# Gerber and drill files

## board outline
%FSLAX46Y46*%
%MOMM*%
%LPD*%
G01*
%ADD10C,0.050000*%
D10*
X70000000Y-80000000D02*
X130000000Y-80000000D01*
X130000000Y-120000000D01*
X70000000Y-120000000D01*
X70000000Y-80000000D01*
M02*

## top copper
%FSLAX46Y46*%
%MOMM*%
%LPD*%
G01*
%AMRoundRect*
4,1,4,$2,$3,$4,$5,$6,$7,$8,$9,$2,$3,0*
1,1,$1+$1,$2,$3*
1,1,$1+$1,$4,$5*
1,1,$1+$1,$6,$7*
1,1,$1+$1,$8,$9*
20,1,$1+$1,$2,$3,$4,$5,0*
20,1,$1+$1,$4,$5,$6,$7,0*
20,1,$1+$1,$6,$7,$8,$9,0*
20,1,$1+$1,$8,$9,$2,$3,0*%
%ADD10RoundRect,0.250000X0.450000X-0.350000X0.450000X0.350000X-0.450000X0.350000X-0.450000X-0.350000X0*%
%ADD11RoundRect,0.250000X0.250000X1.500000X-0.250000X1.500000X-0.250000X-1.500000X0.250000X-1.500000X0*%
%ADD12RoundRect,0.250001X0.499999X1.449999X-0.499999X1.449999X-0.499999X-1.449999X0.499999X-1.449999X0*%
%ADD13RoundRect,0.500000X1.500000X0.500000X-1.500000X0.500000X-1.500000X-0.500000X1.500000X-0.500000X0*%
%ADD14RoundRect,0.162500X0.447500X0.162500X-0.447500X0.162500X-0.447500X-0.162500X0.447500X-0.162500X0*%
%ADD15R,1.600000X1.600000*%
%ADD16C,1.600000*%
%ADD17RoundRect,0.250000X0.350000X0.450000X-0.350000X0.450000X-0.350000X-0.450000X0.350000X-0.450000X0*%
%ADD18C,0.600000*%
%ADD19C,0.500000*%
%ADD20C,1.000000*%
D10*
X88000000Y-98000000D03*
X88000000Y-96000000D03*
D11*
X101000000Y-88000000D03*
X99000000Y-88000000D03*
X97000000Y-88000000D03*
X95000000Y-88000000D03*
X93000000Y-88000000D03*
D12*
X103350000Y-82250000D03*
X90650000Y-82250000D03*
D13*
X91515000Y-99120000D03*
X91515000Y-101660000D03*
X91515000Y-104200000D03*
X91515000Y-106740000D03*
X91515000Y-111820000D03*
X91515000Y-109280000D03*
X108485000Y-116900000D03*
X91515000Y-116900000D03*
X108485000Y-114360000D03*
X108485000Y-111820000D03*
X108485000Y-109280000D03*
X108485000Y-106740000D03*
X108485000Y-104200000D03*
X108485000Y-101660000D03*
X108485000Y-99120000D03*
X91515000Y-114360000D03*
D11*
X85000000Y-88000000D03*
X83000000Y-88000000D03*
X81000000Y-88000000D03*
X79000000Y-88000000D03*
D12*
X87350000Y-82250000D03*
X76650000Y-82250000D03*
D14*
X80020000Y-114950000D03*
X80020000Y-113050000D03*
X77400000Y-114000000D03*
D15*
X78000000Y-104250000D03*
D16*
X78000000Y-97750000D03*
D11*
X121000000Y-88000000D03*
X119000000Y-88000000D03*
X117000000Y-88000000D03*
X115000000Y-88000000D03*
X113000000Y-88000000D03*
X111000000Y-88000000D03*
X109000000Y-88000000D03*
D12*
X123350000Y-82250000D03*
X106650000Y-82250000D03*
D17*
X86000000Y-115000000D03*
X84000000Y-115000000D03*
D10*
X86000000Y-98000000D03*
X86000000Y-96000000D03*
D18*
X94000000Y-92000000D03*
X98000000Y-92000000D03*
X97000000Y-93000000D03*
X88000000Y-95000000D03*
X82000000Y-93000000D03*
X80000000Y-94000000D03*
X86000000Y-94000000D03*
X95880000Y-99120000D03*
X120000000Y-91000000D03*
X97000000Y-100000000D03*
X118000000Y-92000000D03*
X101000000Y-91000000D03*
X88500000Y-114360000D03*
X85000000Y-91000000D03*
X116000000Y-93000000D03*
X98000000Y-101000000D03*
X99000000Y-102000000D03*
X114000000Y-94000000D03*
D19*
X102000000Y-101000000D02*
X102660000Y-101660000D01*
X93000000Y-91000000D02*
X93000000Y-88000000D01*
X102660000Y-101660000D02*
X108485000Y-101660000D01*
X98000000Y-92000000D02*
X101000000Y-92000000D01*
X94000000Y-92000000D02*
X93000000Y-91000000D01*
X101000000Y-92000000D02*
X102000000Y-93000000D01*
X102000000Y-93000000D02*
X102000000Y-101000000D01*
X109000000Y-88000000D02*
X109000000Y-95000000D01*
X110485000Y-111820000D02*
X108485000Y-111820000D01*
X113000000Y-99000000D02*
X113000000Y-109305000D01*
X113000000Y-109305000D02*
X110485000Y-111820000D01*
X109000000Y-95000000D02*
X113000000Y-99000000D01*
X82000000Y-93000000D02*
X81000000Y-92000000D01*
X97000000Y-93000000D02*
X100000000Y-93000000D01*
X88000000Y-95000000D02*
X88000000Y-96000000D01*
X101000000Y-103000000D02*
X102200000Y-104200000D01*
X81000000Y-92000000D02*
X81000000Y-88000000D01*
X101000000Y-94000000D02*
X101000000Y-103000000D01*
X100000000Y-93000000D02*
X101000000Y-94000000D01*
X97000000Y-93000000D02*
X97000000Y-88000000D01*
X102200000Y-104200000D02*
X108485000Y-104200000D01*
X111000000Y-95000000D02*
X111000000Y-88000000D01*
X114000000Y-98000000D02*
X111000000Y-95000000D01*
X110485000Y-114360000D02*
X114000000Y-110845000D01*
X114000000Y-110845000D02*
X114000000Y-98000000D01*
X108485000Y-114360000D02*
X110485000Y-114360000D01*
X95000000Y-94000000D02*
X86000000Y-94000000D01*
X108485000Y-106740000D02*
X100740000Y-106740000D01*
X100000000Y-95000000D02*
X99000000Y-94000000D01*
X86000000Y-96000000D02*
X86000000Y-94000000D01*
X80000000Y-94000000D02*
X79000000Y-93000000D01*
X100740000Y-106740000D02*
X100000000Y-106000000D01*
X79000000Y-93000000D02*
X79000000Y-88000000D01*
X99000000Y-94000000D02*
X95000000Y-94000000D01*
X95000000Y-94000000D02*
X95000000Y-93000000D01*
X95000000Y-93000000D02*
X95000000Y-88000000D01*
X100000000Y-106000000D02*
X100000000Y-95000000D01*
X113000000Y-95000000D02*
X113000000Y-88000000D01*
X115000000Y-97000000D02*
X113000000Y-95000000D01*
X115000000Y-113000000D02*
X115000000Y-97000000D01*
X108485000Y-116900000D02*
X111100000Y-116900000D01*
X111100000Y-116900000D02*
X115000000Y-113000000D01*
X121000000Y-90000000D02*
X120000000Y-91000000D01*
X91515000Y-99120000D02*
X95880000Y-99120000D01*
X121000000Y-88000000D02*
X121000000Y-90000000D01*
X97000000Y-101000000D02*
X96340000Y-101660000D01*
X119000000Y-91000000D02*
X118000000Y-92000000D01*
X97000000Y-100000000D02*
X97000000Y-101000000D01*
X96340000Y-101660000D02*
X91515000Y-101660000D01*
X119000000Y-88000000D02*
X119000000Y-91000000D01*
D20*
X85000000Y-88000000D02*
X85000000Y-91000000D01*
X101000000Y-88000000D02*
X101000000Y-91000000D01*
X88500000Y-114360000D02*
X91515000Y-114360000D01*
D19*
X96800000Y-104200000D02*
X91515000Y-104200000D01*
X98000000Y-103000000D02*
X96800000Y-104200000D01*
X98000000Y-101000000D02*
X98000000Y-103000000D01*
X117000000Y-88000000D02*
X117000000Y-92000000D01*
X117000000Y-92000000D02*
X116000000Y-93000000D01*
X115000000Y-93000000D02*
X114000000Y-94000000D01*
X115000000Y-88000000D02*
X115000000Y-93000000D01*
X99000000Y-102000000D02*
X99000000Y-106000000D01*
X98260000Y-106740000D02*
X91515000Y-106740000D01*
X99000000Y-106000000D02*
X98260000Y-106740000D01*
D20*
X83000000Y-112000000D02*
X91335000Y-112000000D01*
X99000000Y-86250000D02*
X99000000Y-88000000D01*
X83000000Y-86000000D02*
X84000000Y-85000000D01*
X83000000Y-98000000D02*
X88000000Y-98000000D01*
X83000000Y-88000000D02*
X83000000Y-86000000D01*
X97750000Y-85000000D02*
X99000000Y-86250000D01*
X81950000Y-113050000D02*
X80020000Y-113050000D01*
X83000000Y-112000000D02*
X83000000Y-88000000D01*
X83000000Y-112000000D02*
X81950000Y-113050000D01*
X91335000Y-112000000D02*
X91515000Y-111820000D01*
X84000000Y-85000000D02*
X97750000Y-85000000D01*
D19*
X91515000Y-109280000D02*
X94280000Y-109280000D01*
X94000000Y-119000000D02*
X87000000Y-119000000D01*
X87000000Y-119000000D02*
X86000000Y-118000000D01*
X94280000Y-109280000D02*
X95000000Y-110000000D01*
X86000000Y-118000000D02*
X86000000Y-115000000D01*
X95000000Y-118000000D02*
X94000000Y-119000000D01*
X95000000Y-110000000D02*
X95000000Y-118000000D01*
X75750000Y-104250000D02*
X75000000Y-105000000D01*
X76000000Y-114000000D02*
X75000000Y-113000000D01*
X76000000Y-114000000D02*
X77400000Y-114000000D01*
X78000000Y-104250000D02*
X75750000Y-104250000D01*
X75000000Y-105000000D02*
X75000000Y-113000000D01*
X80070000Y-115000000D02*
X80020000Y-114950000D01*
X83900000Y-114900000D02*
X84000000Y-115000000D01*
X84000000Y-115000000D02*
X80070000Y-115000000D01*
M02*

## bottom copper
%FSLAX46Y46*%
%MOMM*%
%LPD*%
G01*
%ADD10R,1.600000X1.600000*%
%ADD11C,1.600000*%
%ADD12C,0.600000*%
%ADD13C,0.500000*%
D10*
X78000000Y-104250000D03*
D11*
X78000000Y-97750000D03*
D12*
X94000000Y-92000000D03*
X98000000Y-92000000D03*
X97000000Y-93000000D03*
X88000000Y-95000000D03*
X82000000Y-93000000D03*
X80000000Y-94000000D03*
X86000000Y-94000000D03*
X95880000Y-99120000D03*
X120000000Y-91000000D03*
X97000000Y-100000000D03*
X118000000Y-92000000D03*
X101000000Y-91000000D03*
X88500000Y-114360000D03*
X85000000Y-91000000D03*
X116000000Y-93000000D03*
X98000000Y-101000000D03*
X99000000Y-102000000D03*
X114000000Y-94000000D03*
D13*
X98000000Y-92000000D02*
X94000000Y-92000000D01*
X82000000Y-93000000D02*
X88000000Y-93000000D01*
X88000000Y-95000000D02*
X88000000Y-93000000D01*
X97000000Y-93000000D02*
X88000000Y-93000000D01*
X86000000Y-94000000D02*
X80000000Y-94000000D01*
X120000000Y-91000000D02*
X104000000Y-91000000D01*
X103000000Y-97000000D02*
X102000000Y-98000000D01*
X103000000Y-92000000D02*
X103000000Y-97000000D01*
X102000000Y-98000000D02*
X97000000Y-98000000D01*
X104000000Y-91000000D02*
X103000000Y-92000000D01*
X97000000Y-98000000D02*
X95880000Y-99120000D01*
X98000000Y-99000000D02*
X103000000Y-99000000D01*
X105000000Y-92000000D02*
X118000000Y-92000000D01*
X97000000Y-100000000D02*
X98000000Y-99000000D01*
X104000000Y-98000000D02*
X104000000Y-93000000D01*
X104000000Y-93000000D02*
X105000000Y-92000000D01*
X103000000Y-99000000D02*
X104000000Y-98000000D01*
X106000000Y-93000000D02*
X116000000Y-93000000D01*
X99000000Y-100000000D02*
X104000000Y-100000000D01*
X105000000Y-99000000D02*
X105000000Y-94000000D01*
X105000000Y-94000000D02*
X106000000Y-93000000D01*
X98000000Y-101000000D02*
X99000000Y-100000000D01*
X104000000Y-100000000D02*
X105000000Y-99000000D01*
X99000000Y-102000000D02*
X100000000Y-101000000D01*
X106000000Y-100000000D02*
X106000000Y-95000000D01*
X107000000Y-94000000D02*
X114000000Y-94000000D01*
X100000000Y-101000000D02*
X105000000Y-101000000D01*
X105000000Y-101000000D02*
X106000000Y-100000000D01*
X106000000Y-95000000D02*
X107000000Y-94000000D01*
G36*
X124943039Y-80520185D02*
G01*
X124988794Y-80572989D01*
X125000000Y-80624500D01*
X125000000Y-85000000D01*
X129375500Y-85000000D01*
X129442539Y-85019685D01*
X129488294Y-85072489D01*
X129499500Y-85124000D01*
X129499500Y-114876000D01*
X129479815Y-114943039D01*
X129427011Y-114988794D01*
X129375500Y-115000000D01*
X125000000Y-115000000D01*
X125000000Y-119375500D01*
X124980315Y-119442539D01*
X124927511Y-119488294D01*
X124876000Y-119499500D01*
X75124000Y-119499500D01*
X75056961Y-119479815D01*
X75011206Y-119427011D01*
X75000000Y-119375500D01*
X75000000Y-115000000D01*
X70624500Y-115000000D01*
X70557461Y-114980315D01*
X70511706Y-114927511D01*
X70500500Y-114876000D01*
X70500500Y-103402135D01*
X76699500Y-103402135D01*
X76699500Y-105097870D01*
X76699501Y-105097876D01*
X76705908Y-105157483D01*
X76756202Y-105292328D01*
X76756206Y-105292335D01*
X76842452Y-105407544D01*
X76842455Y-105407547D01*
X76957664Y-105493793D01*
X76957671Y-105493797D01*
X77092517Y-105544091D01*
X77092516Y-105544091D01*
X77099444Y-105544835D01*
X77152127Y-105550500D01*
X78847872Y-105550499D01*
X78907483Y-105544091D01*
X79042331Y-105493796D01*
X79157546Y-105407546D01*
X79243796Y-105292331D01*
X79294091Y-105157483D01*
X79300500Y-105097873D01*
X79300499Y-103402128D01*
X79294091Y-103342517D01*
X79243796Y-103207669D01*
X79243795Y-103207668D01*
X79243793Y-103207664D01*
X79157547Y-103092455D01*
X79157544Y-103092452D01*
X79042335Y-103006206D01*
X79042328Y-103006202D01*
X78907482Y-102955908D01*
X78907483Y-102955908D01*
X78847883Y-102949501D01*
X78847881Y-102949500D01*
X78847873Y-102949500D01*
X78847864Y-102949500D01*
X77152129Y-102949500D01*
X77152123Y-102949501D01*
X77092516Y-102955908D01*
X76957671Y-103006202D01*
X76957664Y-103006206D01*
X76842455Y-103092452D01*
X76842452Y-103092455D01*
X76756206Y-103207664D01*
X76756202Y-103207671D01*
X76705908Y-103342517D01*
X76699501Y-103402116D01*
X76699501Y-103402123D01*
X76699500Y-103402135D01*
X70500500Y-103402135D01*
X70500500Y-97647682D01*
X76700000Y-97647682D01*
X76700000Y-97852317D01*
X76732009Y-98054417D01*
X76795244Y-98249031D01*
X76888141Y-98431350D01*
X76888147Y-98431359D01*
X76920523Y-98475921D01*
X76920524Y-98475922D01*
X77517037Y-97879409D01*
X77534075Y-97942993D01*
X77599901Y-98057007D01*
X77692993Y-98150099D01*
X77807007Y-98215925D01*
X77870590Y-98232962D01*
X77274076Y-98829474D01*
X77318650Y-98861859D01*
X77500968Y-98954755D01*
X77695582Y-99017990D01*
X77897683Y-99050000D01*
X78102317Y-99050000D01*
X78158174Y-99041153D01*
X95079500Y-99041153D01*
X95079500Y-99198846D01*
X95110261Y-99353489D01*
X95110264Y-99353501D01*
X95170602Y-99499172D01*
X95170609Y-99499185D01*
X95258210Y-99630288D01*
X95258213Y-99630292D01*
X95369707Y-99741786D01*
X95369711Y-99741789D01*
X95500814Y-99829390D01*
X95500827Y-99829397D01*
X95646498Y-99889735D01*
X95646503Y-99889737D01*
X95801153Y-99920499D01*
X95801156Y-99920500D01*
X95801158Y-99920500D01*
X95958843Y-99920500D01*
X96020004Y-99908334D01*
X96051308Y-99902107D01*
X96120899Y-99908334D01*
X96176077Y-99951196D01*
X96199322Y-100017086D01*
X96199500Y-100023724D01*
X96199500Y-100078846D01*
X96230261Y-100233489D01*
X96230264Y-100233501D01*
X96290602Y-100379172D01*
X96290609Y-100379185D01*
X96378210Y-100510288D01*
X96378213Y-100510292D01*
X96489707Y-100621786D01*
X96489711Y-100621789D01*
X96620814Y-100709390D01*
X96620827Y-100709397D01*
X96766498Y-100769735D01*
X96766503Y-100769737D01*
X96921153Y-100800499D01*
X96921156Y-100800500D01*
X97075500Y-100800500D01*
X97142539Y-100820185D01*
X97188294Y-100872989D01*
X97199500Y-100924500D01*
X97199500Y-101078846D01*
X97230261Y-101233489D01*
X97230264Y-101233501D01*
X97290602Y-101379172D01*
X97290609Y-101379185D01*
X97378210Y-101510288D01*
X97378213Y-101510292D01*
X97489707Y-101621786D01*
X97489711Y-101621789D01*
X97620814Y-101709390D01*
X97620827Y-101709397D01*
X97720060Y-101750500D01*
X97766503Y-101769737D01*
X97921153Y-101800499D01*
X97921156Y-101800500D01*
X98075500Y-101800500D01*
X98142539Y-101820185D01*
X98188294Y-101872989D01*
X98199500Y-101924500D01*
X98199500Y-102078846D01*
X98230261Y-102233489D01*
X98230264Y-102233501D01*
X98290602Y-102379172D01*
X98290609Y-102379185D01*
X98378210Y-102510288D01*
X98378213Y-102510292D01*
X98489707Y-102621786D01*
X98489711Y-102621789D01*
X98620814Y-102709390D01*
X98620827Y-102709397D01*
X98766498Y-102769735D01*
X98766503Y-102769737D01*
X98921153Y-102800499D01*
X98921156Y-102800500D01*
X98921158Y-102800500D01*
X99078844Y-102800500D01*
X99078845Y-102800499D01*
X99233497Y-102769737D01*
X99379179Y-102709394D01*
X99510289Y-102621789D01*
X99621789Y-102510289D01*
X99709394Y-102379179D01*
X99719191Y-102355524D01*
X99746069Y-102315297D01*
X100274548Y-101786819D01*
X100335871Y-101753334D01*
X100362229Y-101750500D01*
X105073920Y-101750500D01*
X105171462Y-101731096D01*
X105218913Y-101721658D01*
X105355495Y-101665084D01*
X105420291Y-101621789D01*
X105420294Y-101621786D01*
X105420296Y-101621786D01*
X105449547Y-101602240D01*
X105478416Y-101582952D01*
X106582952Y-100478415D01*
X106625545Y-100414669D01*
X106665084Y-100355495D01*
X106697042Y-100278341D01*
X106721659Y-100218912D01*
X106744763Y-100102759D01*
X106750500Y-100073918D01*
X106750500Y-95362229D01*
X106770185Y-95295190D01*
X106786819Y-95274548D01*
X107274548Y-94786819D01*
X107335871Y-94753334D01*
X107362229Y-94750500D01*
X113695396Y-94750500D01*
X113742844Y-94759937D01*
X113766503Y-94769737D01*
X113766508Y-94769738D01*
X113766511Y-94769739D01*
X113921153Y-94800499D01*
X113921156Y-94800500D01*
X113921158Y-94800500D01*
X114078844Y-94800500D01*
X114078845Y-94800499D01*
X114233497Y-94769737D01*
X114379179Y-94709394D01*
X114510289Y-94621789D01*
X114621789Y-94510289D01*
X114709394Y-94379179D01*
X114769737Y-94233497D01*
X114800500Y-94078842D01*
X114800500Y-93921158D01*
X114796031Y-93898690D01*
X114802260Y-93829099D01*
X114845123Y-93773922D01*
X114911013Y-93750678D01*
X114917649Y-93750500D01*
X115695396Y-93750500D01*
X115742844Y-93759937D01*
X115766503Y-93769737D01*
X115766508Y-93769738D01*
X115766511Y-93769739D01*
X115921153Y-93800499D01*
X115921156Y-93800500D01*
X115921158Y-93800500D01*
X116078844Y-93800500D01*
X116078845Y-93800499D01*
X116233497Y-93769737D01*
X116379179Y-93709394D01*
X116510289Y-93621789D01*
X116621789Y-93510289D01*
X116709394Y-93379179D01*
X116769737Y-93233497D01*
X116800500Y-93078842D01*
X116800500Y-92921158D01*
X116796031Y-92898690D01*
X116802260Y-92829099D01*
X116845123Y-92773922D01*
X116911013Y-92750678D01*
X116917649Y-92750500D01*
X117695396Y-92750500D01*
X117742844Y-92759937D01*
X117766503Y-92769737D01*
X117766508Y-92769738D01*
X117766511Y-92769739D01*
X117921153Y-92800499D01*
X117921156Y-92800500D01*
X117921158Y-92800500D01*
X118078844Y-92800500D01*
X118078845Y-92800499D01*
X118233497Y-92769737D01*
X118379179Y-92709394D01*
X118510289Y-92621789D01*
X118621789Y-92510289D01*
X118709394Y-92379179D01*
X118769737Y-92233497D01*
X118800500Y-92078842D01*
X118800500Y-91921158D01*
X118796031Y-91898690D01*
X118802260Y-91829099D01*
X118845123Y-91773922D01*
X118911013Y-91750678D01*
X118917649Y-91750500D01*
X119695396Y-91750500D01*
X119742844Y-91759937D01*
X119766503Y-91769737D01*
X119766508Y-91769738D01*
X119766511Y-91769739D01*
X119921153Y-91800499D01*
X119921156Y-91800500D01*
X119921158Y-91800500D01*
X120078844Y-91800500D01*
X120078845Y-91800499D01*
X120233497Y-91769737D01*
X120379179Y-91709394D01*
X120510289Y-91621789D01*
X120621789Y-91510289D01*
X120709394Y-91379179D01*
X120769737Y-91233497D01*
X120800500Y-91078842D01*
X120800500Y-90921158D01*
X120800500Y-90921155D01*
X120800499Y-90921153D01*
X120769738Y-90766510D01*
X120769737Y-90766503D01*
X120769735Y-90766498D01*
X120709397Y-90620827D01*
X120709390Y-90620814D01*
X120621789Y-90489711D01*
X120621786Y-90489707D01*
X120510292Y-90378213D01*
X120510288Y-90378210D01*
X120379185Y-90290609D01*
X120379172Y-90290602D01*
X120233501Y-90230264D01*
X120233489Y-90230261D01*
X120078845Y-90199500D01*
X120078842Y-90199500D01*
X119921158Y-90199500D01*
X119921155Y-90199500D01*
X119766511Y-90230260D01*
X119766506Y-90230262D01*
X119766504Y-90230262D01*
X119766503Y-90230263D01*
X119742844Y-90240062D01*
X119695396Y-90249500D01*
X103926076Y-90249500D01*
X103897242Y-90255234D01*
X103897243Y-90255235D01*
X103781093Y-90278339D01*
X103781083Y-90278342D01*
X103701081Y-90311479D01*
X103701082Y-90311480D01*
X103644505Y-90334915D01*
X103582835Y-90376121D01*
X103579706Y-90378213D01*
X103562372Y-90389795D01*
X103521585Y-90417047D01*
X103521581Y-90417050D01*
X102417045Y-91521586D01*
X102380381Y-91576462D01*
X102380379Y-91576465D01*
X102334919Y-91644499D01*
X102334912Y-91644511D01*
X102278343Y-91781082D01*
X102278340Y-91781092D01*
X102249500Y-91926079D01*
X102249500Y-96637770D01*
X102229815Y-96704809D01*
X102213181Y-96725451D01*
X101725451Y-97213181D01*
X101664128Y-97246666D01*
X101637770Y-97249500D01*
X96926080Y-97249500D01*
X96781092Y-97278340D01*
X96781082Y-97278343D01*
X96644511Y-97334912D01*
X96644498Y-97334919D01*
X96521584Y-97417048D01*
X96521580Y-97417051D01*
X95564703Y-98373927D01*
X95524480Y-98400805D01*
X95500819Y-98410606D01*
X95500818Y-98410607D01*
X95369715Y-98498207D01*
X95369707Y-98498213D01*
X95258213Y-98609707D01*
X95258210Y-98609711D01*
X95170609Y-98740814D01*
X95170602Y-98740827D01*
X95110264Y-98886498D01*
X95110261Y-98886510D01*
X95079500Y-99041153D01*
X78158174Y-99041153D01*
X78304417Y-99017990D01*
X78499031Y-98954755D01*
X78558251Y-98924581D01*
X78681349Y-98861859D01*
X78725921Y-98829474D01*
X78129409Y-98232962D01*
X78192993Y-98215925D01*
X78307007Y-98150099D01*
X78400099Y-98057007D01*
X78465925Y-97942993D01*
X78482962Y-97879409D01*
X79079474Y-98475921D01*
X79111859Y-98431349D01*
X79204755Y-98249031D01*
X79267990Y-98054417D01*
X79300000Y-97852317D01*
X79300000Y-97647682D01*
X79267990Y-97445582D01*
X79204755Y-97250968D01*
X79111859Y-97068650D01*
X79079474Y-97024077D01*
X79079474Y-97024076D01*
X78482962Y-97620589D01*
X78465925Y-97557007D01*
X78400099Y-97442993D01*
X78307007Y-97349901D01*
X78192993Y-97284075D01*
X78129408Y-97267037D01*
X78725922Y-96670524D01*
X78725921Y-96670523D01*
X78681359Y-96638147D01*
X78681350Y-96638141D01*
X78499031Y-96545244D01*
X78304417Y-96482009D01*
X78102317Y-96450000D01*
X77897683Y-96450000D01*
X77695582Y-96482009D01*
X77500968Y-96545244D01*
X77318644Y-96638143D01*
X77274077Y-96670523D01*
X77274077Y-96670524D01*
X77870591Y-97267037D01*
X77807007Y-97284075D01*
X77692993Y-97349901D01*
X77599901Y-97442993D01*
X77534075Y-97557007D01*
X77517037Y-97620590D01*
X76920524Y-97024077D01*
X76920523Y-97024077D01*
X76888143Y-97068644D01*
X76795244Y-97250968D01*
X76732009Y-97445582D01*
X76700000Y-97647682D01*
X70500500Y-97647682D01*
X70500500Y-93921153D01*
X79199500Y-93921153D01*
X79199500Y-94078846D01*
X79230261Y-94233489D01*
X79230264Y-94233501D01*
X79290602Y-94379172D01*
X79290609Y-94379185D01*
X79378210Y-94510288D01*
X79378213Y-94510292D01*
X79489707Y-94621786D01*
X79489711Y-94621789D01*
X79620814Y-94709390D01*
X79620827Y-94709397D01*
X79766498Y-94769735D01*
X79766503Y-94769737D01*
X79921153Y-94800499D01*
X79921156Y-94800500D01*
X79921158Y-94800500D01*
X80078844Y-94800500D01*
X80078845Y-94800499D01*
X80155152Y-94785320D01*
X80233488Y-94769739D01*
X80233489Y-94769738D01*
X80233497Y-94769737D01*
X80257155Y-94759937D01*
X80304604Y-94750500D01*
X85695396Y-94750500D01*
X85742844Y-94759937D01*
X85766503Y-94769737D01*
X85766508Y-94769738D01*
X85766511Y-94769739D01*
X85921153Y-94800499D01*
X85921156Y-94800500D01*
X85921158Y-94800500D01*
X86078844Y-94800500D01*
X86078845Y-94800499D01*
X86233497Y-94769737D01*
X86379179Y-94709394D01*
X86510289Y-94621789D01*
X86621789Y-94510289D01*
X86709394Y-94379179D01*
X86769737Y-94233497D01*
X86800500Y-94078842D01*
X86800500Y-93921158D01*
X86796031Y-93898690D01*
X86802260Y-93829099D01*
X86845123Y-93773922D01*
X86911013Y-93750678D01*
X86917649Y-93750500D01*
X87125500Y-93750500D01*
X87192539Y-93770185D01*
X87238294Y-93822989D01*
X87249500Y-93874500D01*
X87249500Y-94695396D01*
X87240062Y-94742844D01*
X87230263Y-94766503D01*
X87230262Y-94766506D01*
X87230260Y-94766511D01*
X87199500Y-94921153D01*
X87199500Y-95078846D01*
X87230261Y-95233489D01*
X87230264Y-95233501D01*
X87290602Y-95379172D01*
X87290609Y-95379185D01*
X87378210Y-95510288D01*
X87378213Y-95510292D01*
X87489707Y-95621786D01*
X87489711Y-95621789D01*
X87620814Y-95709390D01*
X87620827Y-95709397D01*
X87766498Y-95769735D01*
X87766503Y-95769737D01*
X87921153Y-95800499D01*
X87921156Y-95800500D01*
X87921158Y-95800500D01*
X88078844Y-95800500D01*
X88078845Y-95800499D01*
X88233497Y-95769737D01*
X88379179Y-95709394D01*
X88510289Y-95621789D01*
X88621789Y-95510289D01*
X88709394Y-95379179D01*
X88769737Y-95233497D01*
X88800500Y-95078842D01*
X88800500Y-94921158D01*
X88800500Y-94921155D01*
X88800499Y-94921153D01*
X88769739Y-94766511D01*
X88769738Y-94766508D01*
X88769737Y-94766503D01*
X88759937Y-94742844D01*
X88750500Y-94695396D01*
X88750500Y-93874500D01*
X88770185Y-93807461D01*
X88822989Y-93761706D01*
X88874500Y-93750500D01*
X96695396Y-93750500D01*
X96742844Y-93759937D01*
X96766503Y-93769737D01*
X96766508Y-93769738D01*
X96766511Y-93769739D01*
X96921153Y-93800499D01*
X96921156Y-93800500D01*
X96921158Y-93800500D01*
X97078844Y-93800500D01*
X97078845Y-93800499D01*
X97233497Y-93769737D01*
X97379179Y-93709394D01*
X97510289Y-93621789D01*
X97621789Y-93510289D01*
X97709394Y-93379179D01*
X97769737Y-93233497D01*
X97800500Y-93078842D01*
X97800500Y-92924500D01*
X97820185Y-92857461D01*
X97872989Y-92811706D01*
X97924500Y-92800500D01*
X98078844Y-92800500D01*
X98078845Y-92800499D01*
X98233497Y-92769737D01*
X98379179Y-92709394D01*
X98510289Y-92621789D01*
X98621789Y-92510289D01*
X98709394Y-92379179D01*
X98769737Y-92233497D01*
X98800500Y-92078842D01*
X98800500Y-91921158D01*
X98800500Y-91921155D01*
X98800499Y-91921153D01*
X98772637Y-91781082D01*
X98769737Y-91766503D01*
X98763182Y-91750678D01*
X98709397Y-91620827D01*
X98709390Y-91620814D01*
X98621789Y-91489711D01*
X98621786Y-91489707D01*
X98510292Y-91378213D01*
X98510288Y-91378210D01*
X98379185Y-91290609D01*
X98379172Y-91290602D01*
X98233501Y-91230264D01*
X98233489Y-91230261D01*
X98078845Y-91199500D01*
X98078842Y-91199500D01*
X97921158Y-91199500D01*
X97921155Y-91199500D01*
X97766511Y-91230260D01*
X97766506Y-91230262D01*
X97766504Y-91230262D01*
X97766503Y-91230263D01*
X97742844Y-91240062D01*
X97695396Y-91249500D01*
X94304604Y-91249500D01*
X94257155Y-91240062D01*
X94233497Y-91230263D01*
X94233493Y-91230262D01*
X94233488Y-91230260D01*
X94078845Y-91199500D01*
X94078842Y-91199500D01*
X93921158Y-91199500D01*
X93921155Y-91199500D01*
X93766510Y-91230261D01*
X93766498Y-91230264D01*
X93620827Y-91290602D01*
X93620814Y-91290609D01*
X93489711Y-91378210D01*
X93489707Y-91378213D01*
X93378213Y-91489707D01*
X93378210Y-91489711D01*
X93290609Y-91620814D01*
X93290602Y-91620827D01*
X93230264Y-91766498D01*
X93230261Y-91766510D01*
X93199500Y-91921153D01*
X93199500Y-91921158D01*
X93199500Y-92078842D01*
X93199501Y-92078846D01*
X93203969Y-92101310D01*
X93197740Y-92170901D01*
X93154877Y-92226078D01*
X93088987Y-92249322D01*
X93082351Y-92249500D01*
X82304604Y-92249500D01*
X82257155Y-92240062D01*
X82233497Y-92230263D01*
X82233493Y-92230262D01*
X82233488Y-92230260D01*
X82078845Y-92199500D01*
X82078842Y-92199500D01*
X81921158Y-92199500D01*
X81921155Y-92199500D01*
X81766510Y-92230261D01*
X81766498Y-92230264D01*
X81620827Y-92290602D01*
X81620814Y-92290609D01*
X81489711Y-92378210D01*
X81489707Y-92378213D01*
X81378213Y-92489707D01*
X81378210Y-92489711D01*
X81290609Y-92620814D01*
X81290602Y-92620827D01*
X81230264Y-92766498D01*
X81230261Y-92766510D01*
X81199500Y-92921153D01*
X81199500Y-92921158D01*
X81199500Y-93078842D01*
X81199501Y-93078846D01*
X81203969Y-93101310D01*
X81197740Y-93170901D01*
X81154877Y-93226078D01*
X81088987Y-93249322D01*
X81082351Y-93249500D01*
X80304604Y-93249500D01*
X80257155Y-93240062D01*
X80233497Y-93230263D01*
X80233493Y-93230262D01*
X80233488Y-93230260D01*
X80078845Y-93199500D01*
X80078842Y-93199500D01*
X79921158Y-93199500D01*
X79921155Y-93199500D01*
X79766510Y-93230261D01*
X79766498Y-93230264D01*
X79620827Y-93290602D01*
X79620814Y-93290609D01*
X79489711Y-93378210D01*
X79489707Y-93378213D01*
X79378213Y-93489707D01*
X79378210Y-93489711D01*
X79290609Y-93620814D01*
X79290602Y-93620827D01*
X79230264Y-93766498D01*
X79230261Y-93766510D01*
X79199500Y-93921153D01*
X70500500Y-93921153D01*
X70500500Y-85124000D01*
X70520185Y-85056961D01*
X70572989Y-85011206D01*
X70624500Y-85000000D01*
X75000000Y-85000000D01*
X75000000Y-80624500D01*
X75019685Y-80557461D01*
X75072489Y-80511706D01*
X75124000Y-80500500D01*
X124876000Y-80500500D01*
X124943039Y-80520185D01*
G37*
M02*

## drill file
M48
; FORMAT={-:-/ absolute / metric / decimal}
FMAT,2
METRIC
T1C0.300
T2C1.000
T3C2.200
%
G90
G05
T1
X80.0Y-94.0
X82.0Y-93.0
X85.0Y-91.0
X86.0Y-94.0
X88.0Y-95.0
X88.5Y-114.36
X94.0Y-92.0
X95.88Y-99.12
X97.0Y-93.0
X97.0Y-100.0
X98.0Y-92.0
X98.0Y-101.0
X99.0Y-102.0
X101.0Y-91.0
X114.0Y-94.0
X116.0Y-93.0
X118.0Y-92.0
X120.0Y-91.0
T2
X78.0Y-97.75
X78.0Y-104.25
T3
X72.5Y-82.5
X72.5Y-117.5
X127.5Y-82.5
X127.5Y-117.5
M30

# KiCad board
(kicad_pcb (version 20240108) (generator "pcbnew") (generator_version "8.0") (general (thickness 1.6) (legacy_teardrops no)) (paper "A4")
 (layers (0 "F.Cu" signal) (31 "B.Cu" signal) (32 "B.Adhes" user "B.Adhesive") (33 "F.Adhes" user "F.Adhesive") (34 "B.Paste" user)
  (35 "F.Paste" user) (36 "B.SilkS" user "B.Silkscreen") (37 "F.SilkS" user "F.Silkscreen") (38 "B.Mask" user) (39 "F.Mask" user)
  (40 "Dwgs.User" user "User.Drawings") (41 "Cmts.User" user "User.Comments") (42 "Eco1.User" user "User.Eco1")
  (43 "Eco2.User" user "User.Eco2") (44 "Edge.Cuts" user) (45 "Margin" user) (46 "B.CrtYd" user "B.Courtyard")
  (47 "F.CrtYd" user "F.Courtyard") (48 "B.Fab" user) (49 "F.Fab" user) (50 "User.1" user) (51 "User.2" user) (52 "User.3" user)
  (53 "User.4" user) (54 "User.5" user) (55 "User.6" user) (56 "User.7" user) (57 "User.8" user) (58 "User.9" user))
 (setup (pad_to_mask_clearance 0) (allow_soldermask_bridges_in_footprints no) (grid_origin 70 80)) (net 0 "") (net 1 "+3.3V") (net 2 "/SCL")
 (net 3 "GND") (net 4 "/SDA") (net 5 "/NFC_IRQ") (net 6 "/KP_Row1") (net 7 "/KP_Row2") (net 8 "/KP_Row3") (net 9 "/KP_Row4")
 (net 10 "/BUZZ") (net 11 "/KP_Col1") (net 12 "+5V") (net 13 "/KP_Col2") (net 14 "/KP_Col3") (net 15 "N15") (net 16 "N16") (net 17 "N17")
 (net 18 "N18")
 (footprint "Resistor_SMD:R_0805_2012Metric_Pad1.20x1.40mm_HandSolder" (layer "F.Cu") (at 88 97 90)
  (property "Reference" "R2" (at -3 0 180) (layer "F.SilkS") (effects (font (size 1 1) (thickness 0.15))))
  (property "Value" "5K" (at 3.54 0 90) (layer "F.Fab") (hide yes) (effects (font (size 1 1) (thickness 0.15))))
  (pad "1" smd roundrect (at -1 0 90) (size 1.2 1.4) (layers "F.Cu" "F.Paste" "F.Mask") (roundrect_rratio 0.208333) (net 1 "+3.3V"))
  (pad "2" smd roundrect (at 1 0 90) (size 1.2 1.4) (layers "F.Cu" "F.Paste" "F.Mask") (roundrect_rratio 0.208333) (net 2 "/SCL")))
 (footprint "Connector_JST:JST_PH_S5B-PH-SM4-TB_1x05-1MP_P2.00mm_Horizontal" (layer "F.Cu") (at 97 85.15 180)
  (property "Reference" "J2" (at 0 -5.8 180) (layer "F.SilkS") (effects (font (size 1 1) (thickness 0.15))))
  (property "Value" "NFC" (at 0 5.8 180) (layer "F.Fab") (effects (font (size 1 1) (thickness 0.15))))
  (pad "1" smd roundrect (at -4 -2.85 180) (size 1 3.5) (layers "F.Cu" "F.Paste" "F.Mask") (roundrect_rratio 0.25) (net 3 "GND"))
  (pad "2" smd roundrect (at -2 -2.85 180) (size 1 3.5) (layers "F.Cu" "F.Paste" "F.Mask") (roundrect_rratio 0.25) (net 1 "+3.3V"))
  (pad "3" smd roundrect (at 0 -2.85 180) (size 1 3.5) (layers "F.Cu" "F.Paste" "F.Mask") (roundrect_rratio 0.25) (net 2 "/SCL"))
  (pad "4" smd roundrect (at 2 -2.85 180) (size 1 3.5) (layers "F.Cu" "F.Paste" "F.Mask") (roundrect_rratio 0.25) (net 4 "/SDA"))
  (pad "5" smd roundrect (at 4 -2.85 180) (size 1 3.5) (layers "F.Cu" "F.Paste" "F.Mask") (roundrect_rratio 0.25) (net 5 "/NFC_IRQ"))
  (pad "MP" smd roundrect (at -6.35 2.9 180) (size 1.5 3.4) (layers "F.Cu" "F.Paste" "F.Mask") (roundrect_rratio 0.166667))
  (pad "MP" smd roundrect (at 6.35 2.9 180) (size 1.5 3.4) (layers "F.Cu" "F.Paste" "F.Mask") (roundrect_rratio 0.166667)))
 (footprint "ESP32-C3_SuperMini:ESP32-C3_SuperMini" (layer "F.Cu") (at 100 107 180)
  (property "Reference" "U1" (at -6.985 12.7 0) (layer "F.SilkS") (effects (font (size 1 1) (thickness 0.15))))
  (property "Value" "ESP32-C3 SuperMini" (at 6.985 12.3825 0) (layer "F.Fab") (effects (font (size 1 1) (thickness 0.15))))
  (pad "0" smd roundrect (at 8.485 7.88 180) (size 4 2) (layers "F.Cu" "F.Paste" "F.Mask") (roundrect_rratio 0.25) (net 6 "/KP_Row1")
   (solder_mask_margin 0.102))
  (pad "1" smd roundrect (at 8.485 5.34 180) (size 4 2) (layers "F.Cu" "F.Paste" "F.Mask") (roundrect_rratio 0.25) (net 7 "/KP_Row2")
   (solder_mask_margin 0.102))
  (pad "2" smd roundrect (at 8.485 2.8 180) (size 4 2) (layers "F.Cu" "F.Paste" "F.Mask") (roundrect_rratio 0.25) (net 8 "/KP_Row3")
   (solder_mask_margin 0.102))
  (pad "3" smd roundrect (at 8.485 0.26 180) (size 4 2) (layers "F.Cu" "F.Paste" "F.Mask") (roundrect_rratio 0.25) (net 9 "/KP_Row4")
   (solder_mask_margin 0.102))
  (pad "3.3" smd roundrect (at 8.485 -4.82 180) (size 4 2) (layers "F.Cu" "F.Paste" "F.Mask") (roundrect_rratio 0.25) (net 1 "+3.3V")
   (solder_mask_margin 0.102))
  (pad "4" smd roundrect (at 8.485 -2.28 180) (size 4 2) (layers "F.Cu" "F.Paste" "F.Mask") (roundrect_rratio 0.25) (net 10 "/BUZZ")
   (solder_mask_margin 0.102))
  (pad "5" smd roundrect (at -8.485 -9.9 180) (size 4 2) (layers "F.Cu" "F.Paste" "F.Mask") (roundrect_rratio 0.25) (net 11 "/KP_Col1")
   (solder_mask_margin 0.102))
  (pad "5V" smd roundrect (at 8.485 -9.9 180) (size 4 2) (layers "F.Cu" "F.Paste" "F.Mask") (roundrect_rratio 0.25) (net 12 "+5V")
   (solder_mask_margin 0.102))
  (pad "6" smd roundrect (at -8.485 -7.36 180) (size 4 2) (layers "F.Cu" "F.Paste" "F.Mask") (roundrect_rratio 0.25) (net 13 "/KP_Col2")
   (solder_mask_margin 0.102))
  (pad "7" smd roundrect (at -8.485 -4.82 180) (size 4 2) (layers "F.Cu" "F.Paste" "F.Mask") (roundrect_rratio 0.25) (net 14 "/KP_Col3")
   (solder_mask_margin 0.102))
  (pad "8" smd roundrect (at -8.485 -2.28 180) (size 4 2) (layers "F.Cu" "F.Paste" "F.Mask") (roundrect_rratio 0.25) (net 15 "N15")
   (solder_mask_margin 0.102))
  (pad "9" smd roundrect (at -8.485 0.26 180) (size 4 2) (layers "F.Cu" "F.Paste" "F.Mask") (roundrect_rratio 0.25) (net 4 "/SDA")
   (solder_mask_margin 0.102))
  (pad "10" smd roundrect (at -8.485 2.8 180) (size 4 2) (layers "F.Cu" "F.Paste" "F.Mask") (roundrect_rratio 0.25) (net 2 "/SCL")
   (solder_mask_margin 0.102))
  (pad "20" smd roundrect (at -8.485 5.34 180) (size 4 2) (layers "F.Cu" "F.Paste" "F.Mask") (roundrect_rratio 0.25) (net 5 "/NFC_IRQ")
   (solder_mask_margin 0.102))
  (pad "21" smd roundrect (at -8.485 7.88 180) (size 4 2) (layers "F.Cu" "F.Paste" "F.Mask") (roundrect_rratio 0.25) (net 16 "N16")
   (solder_mask_margin 0.102))
  (pad "G" smd roundrect (at 8.485 -7.36 180) (size 4 2) (layers "F.Cu" "F.Paste" "F.Mask") (roundrect_rratio 0.25) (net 3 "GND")
   (solder_mask_margin 0.102))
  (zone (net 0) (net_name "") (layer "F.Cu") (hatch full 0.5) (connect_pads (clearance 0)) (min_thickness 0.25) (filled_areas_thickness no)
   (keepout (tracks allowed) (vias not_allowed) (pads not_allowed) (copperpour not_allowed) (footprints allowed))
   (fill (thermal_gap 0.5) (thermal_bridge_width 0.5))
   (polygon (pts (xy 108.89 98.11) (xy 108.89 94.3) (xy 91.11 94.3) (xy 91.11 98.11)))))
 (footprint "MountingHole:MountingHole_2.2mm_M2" (layer "F.Cu") (at 72.5 82.5)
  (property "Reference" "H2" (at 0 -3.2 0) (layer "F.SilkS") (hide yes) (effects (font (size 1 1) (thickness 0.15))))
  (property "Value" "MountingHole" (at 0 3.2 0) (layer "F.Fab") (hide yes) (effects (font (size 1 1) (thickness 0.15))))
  (pad "" np_thru_hole circle (at 0 0) (size 2.2 2.2) (drill 2.2) (layers "*.Cu" "*.Mask")))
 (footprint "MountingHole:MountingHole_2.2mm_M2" (layer "F.Cu") (at 72.5 117.5)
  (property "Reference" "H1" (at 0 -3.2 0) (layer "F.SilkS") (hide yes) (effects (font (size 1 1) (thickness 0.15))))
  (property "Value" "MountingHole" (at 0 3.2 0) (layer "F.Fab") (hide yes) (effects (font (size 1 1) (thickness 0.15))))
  (pad "" np_thru_hole circle (at 0 0) (size 2.2 2.2) (drill 2.2) (layers "*.Cu" "*.Mask")))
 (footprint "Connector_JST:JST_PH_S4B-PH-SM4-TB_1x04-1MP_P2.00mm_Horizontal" (layer "F.Cu") (at 82 85.15 180)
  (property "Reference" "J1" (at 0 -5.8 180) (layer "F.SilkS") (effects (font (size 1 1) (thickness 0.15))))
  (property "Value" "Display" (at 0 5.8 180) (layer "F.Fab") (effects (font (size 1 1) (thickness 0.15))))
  (pad "1" smd roundrect (at -3 -2.85 180) (size 1 3.5) (layers "F.Cu" "F.Paste" "F.Mask") (roundrect_rratio 0.25) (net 3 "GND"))
  (pad "2" smd roundrect (at -1 -2.85 180) (size 1 3.5) (layers "F.Cu" "F.Paste" "F.Mask") (roundrect_rratio 0.25) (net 1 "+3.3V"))
  (pad "3" smd roundrect (at 1 -2.85 180) (size 1 3.5) (layers "F.Cu" "F.Paste" "F.Mask") (roundrect_rratio 0.25) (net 2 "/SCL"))
  (pad "4" smd roundrect (at 3 -2.85 180) (size 1 3.5) (layers "F.Cu" "F.Paste" "F.Mask") (roundrect_rratio 0.25) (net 4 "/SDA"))
  (pad "MP" smd roundrect (at -5.35 2.9 180) (size 1.5 3.4) (layers "F.Cu" "F.Paste" "F.Mask") (roundrect_rratio 0.166667))
  (pad "MP" smd roundrect (at 5.35 2.9 180) (size 1.5 3.4) (layers "F.Cu" "F.Paste" "F.Mask") (roundrect_rratio 0.166667)))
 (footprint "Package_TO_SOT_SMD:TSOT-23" (layer "F.Cu") (at 78.71 114 180)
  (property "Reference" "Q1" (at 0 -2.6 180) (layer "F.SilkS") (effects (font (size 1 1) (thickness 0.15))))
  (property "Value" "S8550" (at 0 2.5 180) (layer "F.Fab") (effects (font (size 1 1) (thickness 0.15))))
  (pad "1" smd roundrect (at -1.31 -0.95 180) (size 1.22 0.65) (layers "F.Cu" "F.Paste" "F.Mask") (roundrect_rratio 0.25) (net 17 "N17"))
  (pad "2" smd roundrect (at -1.31 0.95 180) (size 1.22 0.65) (layers "F.Cu" "F.Paste" "F.Mask") (roundrect_rratio 0.25) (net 1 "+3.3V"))
  (pad "3" smd roundrect (at 1.31 0 180) (size 1.22 0.65) (layers "F.Cu" "F.Paste" "F.Mask") (roundrect_rratio 0.25) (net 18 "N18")))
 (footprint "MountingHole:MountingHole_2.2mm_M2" (layer "F.Cu") (at 127.5 117.5)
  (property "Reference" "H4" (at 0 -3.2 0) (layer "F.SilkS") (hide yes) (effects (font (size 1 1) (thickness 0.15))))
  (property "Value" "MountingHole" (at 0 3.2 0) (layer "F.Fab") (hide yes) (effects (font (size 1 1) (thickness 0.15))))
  (pad "" np_thru_hole circle (at 0 0) (size 2.2 2.2) (drill 2.2) (layers "*.Cu" "*.Mask")))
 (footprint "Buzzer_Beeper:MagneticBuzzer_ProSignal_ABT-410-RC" (layer "F.Cu") (at 78 104.25 90)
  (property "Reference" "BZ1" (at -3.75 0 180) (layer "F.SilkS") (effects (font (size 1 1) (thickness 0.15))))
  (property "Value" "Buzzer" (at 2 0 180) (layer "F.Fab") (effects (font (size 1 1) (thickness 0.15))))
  (pad "1" thru_hole rect (at 0 0 90) (size 1.6 1.6) (drill 1) (layers "*.Cu" "*.Mask") (remove_unused_layers no) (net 18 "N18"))
  (pad "2" thru_hole circle (at 6.5 0 90) (size 1.6 1.6) (drill 1) (layers "*.Cu" "*.Mask") (remove_unused_layers no) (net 3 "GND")))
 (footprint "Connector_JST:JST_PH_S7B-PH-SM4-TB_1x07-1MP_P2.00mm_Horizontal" (layer "F.Cu") (at 115 85.15 180)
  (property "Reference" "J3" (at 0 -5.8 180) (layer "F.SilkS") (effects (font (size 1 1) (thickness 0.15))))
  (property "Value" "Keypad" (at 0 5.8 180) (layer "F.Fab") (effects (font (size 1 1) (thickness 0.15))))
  (pad "1" smd roundrect (at -6 -2.85 180) (size 1 3.5) (layers "F.Cu" "F.Paste" "F.Mask") (roundrect_rratio 0.25) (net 6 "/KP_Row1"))
  (pad "2" smd roundrect (at -4 -2.85 180) (size 1 3.5) (layers "F.Cu" "F.Paste" "F.Mask") (roundrect_rratio 0.25) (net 7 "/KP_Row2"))
  (pad "3" smd roundrect (at -2 -2.85 180) (size 1 3.5) (layers "F.Cu" "F.Paste" "F.Mask") (roundrect_rratio 0.25) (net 8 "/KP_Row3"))
  (pad "4" smd roundrect (at 0 -2.85 180) (size 1 3.5) (layers "F.Cu" "F.Paste" "F.Mask") (roundrect_rratio 0.25) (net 9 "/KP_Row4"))
  (pad "5" smd roundrect (at 2 -2.85 180) (size 1 3.5) (layers "F.Cu" "F.Paste" "F.Mask") (roundrect_rratio 0.25) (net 11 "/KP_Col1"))
  (pad "6" smd roundrect (at 4 -2.85 180) (size 1 3.5) (layers "F.Cu" "F.Paste" "F.Mask") (roundrect_rratio 0.25) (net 13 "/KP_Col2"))
  (pad "7" smd roundrect (at 6 -2.85 180) (size 1 3.5) (layers "F.Cu" "F.Paste" "F.Mask") (roundrect_rratio 0.25) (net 14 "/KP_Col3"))
  (pad "MP" smd roundrect (at -8.35 2.9 180) (size 1.5 3.4) (layers "F.Cu" "F.Paste" "F.Mask") (roundrect_rratio 0.166667))
  (pad "MP" smd roundrect (at 8.35 2.9 180) (size 1.5 3.4) (layers "F.Cu" "F.Paste" "F.Mask") (roundrect_rratio 0.166667)))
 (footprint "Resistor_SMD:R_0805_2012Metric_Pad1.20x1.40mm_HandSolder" (layer "F.Cu") (at 85 115 180)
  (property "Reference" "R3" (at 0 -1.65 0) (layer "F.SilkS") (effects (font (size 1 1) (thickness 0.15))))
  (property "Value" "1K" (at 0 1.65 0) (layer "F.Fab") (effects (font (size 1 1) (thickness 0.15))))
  (pad "1" smd roundrect (at -1 0 180) (size 1.2 1.4) (layers "F.Cu" "F.Paste" "F.Mask") (roundrect_rratio 0.208333) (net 10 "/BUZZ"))
  (pad "2" smd roundrect (at 1 0 180) (size 1.2 1.4) (layers "F.Cu" "F.Paste" "F.Mask") (roundrect_rratio 0.208333) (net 17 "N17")))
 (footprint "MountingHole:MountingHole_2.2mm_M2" (layer "F.Cu") (at 127.5 82.5)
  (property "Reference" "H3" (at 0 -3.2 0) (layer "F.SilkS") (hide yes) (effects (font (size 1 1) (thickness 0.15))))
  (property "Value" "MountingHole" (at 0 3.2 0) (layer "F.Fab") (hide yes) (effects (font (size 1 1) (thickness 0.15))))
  (pad "" np_thru_hole circle (at 0 0) (size 2.2 2.2) (drill 2.2) (layers "*.Cu" "*.Mask")))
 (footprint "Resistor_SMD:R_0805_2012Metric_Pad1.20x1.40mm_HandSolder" (layer "F.Cu") (at 86 97 90)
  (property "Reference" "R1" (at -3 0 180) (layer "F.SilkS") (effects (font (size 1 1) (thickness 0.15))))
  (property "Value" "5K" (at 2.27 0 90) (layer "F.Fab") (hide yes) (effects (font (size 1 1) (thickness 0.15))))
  (pad "1" smd roundrect (at -1 0 90) (size 1.2 1.4) (layers "F.Cu" "F.Paste" "F.Mask") (roundrect_rratio 0.208333) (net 1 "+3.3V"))
  (pad "2" smd roundrect (at 1 0 90) (size 1.2 1.4) (layers "F.Cu" "F.Paste" "F.Mask") (roundrect_rratio 0.208333) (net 4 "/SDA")))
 (gr_rect (start 70 80) (end 130 120) (stroke (width 0.05) (type default)) (fill none) (layer "Edge.Cuts"))
 (segment (start 102 101) (end 102.66 101.66) (width 0.5) (layer "F.Cu") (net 5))
 (segment (start 93 91) (end 93 88) (width 0.5) (layer "F.Cu") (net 5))
 (segment (start 102.66 101.66) (end 108.485 101.66) (width 0.5) (layer "F.Cu") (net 5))
 (segment (start 98 92) (end 101 92) (width 0.5) (layer "F.Cu") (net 5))
 (segment (start 94 92) (end 93 91) (width 0.5) (layer "F.Cu") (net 5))
 (segment (start 101 92) (end 102 93) (width 0.5) (layer "F.Cu") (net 5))
 (segment (start 102 93) (end 102 101) (width 0.5) (layer "F.Cu") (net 5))
 (via (at 94 92) (size 0.6) (drill 0.3) (layers "F.Cu" "B.Cu") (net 5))
 (via (at 98 92) (size 0.6) (drill 0.3) (layers "F.Cu" "B.Cu") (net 5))
 (segment (start 98 92) (end 94 92) (width 0.5) (layer "B.Cu") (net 5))
 (segment (start 109 88) (end 109 95) (width 0.5) (layer "F.Cu") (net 14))
 (segment (start 110.485 111.82) (end 108.485 111.82) (width 0.5) (layer "F.Cu") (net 14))
 (segment (start 113 99) (end 113 109.305) (width 0.5) (layer "F.Cu") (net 14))
 (segment (start 113 109.305) (end 110.485 111.82) (width 0.5) (layer "F.Cu") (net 14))
 (segment (start 109 95) (end 113 99) (width 0.5) (layer "F.Cu") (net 14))
 (segment (start 82 93) (end 81 92) (width 0.5) (layer "F.Cu") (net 2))
 (segment (start 97 93) (end 100 93) (width 0.5) (layer "F.Cu") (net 2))
 (segment (start 88 95) (end 88 96) (width 0.5) (layer "F.Cu") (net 2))
 (segment (start 101 103) (end 102.2 104.2) (width 0.5) (layer "F.Cu") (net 2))
 (segment (start 81 92) (end 81 88) (width 0.5) (layer "F.Cu") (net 2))
 (segment (start 101 94) (end 101 103) (width 0.5) (layer "F.Cu") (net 2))
 (segment (start 100 93) (end 101 94) (width 0.5) (layer "F.Cu") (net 2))
 (segment (start 97 93) (end 97 88) (width 0.5) (layer "F.Cu") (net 2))
 (segment (start 102.2 104.2) (end 108.485 104.2) (width 0.5) (layer "F.Cu") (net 2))
 (via (at 97 93) (size 0.6) (drill 0.3) (layers "F.Cu" "B.Cu") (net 2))
 (via (at 88 95) (size 0.6) (drill 0.3) (layers "F.Cu" "B.Cu") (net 2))
 (via (at 82 93) (size 0.6) (drill 0.3) (layers "F.Cu" "B.Cu") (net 2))
 (segment (start 82 93) (end 88 93) (width 0.5) (layer "B.Cu") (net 2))
 (segment (start 88 95) (end 88 93) (width 0.5) (layer "B.Cu") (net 2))
 (segment (start 97 93) (end 88 93) (width 0.5) (layer "B.Cu") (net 2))
 (segment (start 111 95) (end 111 88) (width 0.5) (layer "F.Cu") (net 13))
 (segment (start 114 98) (end 111 95) (width 0.5) (layer "F.Cu") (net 13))
 (segment (start 110.485 114.36) (end 114 110.845) (width 0.5) (layer "F.Cu") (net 13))
 (segment (start 114 110.845) (end 114 98) (width 0.5) (layer "F.Cu") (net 13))
 (segment (start 108.485 114.36) (end 110.485 114.36) (width 0.5) (layer "F.Cu") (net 13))
 (segment (start 95 94) (end 86 94) (width 0.5) (layer "F.Cu") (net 4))
 (segment (start 108.485 106.74) (end 100.74 106.74) (width 0.5) (layer "F.Cu") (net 4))
 (segment (start 100 95) (end 99 94) (width 0.5) (layer "F.Cu") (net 4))
 (segment (start 86 96) (end 86 94) (width 0.5) (layer "F.Cu") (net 4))
 (segment (start 80 94) (end 79 93) (width 0.5) (layer "F.Cu") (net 4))
 (segment (start 100.74 106.74) (end 100 106) (width 0.5) (layer "F.Cu") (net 4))
 (segment (start 79 93) (end 79 88) (width 0.5) (layer "F.Cu") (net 4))
 (segment (start 99 94) (end 95 94) (width 0.5) (layer "F.Cu") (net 4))
 (segment (start 95 94) (end 95 93) (width 0.5) (layer "F.Cu") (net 4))
 (segment (start 95 93) (end 95 88) (width 0.5) (layer "F.Cu") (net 4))
 (segment (start 100 106) (end 100 95) (width 0.5) (layer "F.Cu") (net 4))
 (via (at 80 94) (size 0.6) (drill 0.3) (layers "F.Cu" "B.Cu") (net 4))
 (via (at 86 94) (size 0.6) (drill 0.3) (layers "F.Cu" "B.Cu") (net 4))
 (segment (start 86 94) (end 80 94) (width 0.5) (layer "B.Cu") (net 4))
 (segment (start 113 95) (end 113 88) (width 0.5) (layer "F.Cu") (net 11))
 (segment (start 115 97) (end 113 95) (width 0.5) (layer "F.Cu") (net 11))
 (segment (start 115 113) (end 115 97) (width 0.5) (layer "F.Cu") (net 11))
 (segment (start 108.485 116.9) (end 111.1 116.9) (width 0.5) (layer "F.Cu") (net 11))
 (segment (start 111.1 116.9) (end 115 113) (width 0.5) (layer "F.Cu") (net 11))
 (segment (start 121 90) (end 120 91) (width 0.5) (layer "F.Cu") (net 6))
 (segment (start 91.515 99.12) (end 95.88 99.12) (width 0.5) (layer "F.Cu") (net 6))
 (segment (start 121 88) (end 121 90) (width 0.5) (layer "F.Cu") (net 6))
 (via (at 95.88 99.12) (size 0.6) (drill 0.3) (layers "F.Cu" "B.Cu") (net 6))
 (via (at 120 91) (size 0.6) (drill 0.3) (layers "F.Cu" "B.Cu") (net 6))
 (segment (start 120 91) (end 104 91) (width 0.5) (layer "B.Cu") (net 6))
 (segment (start 103 97) (end 102 98) (width 0.5) (layer "B.Cu") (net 6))
 (segment (start 103 92) (end 103 97) (width 0.5) (layer "B.Cu") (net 6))
 (segment (start 102 98) (end 97 98) (width 0.5) (layer "B.Cu") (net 6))
 (segment (start 104 91) (end 103 92) (width 0.5) (layer "B.Cu") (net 6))
 (segment (start 97 98) (end 95.88 99.12) (width 0.5) (layer "B.Cu") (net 6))
 (segment (start 97 101) (end 96.34 101.66) (width 0.5) (layer "F.Cu") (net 7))
 (segment (start 119 91) (end 118 92) (width 0.5) (layer "F.Cu") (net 7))
 (segment (start 97 100) (end 97 101) (width 0.5) (layer "F.Cu") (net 7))
 (segment (start 96.34 101.66) (end 91.515 101.66) (width 0.5) (layer "F.Cu") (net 7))
 (segment (start 119 88) (end 119 91) (width 0.5) (layer "F.Cu") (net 7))
 (via (at 97 100) (size 0.6) (drill 0.3) (layers "F.Cu" "B.Cu") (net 7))
 (via (at 118 92) (size 0.6) (drill 0.3) (layers "F.Cu" "B.Cu") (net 7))
 (segment (start 98 99) (end 103 99) (width 0.5) (layer "B.Cu") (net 7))
 (segment (start 105 92) (end 118 92) (width 0.5) (layer "B.Cu") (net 7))
 (segment (start 97 100) (end 98 99) (width 0.5) (layer "B.Cu") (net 7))
 (segment (start 104 98) (end 104 93) (width 0.5) (layer "B.Cu") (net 7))
 (segment (start 104 93) (end 105 92) (width 0.5) (layer "B.Cu") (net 7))
 (segment (start 103 99) (end 104 98) (width 0.5) (layer "B.Cu") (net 7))
 (segment (start 85 88) (end 85 91) (width 1) (layer "F.Cu") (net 3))
 (segment (start 101 88) (end 101 91) (width 1) (layer "F.Cu") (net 3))
 (segment (start 88.5 114.36) (end 91.515 114.36) (width 1) (layer "F.Cu") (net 3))
 (via (at 101 91) (size 0.6) (drill 0.3) (layers "F.Cu" "B.Cu") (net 3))
 (via (at 88.5 114.36) (size 0.6) (drill 0.3) (layers "F.Cu" "B.Cu") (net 3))
 (via (at 85 91) (size 0.6) (drill 0.3) (layers "F.Cu" "B.Cu") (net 3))
 (segment (start 96.8 104.2) (end 91.515 104.2) (width 0.5) (layer "F.Cu") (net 8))
 (segment (start 98 103) (end 96.8 104.2) (width 0.5) (layer "F.Cu") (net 8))
 (segment (start 98 101) (end 98 103) (width 0.5) (layer "F.Cu") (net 8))
 (segment (start 117 88) (end 117 92) (width 0.5) (layer "F.Cu") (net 8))
 (segment (start 117 92) (end 116 93) (width 0.5) (layer "F.Cu") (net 8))
 (via (at 116 93) (size 0.6) (drill 0.3) (layers "F.Cu" "B.Cu") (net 8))
 (via (at 98 101) (size 0.6) (drill 0.3) (layers "F.Cu" "B.Cu") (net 8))
 (segment (start 106 93) (end 116 93) (width 0.5) (layer "B.Cu") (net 8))
 (segment (start 99 100) (end 104 100) (width 0.5) (layer "B.Cu") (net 8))
 (segment (start 105 99) (end 105 94) (width 0.5) (layer "B.Cu") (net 8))
 (segment (start 105 94) (end 106 93) (width 0.5) (layer "B.Cu") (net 8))
 (segment (start 98 101) (end 99 100) (width 0.5) (layer "B.Cu") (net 8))
 (segment (start 104 100) (end 105 99) (width 0.5) (layer "B.Cu") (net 8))
 (segment (start 115 93) (end 114 94) (width 0.5) (layer "F.Cu") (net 9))
 (segment (start 115 88) (end 115 93) (width 0.5) (layer "F.Cu") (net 9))
 (segment (start 99 102) (end 99 106) (width 0.5) (layer "F.Cu") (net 9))
 (segment (start 98.26 106.74) (end 91.515 106.74) (width 0.5) (layer "F.Cu") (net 9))
 (segment (start 99 106) (end 98.26 106.74) (width 0.5) (layer "F.Cu") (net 9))
 (via (at 99 102) (size 0.6) (drill 0.3) (layers "F.Cu" "B.Cu") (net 9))
 (via (at 114 94) (size 0.6) (drill 0.3) (layers "F.Cu" "B.Cu") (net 9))
 (segment (start 99 102) (end 100 101) (width 0.5) (layer "B.Cu") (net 9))
 (segment (start 106 100) (end 106 95) (width 0.5) (layer "B.Cu") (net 9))
 (segment (start 107 94) (end 114 94) (width 0.5) (layer "B.Cu") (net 9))
 (segment (start 100 101) (end 105 101) (width 0.5) (layer "B.Cu") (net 9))
 (segment (start 105 101) (end 106 100) (width 0.5) (layer "B.Cu") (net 9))
 (segment (start 106 95) (end 107 94) (width 0.5) (layer "B.Cu") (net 9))
 (segment (start 83 112) (end 91.335 112) (width 1) (layer "F.Cu") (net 1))
 (segment (start 99 86.25) (end 99 88) (width 1) (layer "F.Cu") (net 1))
 (segment (start 83 86) (end 84 85) (width 1) (layer "F.Cu") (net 1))
 (segment (start 83 98) (end 88 98) (width 1) (layer "F.Cu") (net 1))
 (segment (start 83 88) (end 83 86) (width 1) (layer "F.Cu") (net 1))
 (segment (start 97.75 85) (end 99 86.25) (width 1) (layer "F.Cu") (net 1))
 (segment (start 81.95 113.05) (end 80.02 113.05) (width 1) (layer "F.Cu") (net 1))
 (segment (start 83 112) (end 83 88) (width 1) (layer "F.Cu") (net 1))
 (segment (start 83 112) (end 81.95 113.05) (width 1) (layer "F.Cu") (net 1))
 (segment (start 91.335 112) (end 91.515 111.82) (width 1) (layer "F.Cu") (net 1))
 (segment (start 84 85) (end 97.75 85) (width 1) (layer "F.Cu") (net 1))
 (segment (start 91.515 109.28) (end 94.28 109.28) (width 0.5) (layer "F.Cu") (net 10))
 (segment (start 94 119) (end 87 119) (width 0.5) (layer "F.Cu") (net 10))
 (segment (start 87 119) (end 86 118) (width 0.5) (layer "F.Cu") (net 10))
 (segment (start 94.28 109.28) (end 95 110) (width 0.5) (layer "F.Cu") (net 10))
 (segment (start 86 118) (end 86 115) (width 0.5) (layer "F.Cu") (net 10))
 (segment (start 95 118) (end 94 119) (width 0.5) (layer "F.Cu") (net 10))
 (segment (start 95 110) (end 95 118) (width 0.5) (layer "F.Cu") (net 10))
 (segment (start 75.75 104.25) (end 75 105) (width 0.5) (layer "F.Cu") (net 18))
 (segment (start 76 114) (end 75 113) (width 0.5) (layer "F.Cu") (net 18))
 (segment (start 76 114) (end 77.4 114) (width 0.5) (layer "F.Cu") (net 18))
 (segment (start 78 104.25) (end 75.75 104.25) (width 0.5) (layer "F.Cu") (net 18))
 (segment (start 75 105) (end 75 113) (width 0.5) (layer "F.Cu") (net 18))
 (segment (start 80.07 115) (end 80.02 114.95) (width 0.5) (layer "F.Cu") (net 17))
 (segment (start 83.9 114.9) (end 84 115) (width 0.5) (layer "F.Cu") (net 17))
 (segment (start 84 115) (end 80.07 115) (width 0.5) (layer "F.Cu") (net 17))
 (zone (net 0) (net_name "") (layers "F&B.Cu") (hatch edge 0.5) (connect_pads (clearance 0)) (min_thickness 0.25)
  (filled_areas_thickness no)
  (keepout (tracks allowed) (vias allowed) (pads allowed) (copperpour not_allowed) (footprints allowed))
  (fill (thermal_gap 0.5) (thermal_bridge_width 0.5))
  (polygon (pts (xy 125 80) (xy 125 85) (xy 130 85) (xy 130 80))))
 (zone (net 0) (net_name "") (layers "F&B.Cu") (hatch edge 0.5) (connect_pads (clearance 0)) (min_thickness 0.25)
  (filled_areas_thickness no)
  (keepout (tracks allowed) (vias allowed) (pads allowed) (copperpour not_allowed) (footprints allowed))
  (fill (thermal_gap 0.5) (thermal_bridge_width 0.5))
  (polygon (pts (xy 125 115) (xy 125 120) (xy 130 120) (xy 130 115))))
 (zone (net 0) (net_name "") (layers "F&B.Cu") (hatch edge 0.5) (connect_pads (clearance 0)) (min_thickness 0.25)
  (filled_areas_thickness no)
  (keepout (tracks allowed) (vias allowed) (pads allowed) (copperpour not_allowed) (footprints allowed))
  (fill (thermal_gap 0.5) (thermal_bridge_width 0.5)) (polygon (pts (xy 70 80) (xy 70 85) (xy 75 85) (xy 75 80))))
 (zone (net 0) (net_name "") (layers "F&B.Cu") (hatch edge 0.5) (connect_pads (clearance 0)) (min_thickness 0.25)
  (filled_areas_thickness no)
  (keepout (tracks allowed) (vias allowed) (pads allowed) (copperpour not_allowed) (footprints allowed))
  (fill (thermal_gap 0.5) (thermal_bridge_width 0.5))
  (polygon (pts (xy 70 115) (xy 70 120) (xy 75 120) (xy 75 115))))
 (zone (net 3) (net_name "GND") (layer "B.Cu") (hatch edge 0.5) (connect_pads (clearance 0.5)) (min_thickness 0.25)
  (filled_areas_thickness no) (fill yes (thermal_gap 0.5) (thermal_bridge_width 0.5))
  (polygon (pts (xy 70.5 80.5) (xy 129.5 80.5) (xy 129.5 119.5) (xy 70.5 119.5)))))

